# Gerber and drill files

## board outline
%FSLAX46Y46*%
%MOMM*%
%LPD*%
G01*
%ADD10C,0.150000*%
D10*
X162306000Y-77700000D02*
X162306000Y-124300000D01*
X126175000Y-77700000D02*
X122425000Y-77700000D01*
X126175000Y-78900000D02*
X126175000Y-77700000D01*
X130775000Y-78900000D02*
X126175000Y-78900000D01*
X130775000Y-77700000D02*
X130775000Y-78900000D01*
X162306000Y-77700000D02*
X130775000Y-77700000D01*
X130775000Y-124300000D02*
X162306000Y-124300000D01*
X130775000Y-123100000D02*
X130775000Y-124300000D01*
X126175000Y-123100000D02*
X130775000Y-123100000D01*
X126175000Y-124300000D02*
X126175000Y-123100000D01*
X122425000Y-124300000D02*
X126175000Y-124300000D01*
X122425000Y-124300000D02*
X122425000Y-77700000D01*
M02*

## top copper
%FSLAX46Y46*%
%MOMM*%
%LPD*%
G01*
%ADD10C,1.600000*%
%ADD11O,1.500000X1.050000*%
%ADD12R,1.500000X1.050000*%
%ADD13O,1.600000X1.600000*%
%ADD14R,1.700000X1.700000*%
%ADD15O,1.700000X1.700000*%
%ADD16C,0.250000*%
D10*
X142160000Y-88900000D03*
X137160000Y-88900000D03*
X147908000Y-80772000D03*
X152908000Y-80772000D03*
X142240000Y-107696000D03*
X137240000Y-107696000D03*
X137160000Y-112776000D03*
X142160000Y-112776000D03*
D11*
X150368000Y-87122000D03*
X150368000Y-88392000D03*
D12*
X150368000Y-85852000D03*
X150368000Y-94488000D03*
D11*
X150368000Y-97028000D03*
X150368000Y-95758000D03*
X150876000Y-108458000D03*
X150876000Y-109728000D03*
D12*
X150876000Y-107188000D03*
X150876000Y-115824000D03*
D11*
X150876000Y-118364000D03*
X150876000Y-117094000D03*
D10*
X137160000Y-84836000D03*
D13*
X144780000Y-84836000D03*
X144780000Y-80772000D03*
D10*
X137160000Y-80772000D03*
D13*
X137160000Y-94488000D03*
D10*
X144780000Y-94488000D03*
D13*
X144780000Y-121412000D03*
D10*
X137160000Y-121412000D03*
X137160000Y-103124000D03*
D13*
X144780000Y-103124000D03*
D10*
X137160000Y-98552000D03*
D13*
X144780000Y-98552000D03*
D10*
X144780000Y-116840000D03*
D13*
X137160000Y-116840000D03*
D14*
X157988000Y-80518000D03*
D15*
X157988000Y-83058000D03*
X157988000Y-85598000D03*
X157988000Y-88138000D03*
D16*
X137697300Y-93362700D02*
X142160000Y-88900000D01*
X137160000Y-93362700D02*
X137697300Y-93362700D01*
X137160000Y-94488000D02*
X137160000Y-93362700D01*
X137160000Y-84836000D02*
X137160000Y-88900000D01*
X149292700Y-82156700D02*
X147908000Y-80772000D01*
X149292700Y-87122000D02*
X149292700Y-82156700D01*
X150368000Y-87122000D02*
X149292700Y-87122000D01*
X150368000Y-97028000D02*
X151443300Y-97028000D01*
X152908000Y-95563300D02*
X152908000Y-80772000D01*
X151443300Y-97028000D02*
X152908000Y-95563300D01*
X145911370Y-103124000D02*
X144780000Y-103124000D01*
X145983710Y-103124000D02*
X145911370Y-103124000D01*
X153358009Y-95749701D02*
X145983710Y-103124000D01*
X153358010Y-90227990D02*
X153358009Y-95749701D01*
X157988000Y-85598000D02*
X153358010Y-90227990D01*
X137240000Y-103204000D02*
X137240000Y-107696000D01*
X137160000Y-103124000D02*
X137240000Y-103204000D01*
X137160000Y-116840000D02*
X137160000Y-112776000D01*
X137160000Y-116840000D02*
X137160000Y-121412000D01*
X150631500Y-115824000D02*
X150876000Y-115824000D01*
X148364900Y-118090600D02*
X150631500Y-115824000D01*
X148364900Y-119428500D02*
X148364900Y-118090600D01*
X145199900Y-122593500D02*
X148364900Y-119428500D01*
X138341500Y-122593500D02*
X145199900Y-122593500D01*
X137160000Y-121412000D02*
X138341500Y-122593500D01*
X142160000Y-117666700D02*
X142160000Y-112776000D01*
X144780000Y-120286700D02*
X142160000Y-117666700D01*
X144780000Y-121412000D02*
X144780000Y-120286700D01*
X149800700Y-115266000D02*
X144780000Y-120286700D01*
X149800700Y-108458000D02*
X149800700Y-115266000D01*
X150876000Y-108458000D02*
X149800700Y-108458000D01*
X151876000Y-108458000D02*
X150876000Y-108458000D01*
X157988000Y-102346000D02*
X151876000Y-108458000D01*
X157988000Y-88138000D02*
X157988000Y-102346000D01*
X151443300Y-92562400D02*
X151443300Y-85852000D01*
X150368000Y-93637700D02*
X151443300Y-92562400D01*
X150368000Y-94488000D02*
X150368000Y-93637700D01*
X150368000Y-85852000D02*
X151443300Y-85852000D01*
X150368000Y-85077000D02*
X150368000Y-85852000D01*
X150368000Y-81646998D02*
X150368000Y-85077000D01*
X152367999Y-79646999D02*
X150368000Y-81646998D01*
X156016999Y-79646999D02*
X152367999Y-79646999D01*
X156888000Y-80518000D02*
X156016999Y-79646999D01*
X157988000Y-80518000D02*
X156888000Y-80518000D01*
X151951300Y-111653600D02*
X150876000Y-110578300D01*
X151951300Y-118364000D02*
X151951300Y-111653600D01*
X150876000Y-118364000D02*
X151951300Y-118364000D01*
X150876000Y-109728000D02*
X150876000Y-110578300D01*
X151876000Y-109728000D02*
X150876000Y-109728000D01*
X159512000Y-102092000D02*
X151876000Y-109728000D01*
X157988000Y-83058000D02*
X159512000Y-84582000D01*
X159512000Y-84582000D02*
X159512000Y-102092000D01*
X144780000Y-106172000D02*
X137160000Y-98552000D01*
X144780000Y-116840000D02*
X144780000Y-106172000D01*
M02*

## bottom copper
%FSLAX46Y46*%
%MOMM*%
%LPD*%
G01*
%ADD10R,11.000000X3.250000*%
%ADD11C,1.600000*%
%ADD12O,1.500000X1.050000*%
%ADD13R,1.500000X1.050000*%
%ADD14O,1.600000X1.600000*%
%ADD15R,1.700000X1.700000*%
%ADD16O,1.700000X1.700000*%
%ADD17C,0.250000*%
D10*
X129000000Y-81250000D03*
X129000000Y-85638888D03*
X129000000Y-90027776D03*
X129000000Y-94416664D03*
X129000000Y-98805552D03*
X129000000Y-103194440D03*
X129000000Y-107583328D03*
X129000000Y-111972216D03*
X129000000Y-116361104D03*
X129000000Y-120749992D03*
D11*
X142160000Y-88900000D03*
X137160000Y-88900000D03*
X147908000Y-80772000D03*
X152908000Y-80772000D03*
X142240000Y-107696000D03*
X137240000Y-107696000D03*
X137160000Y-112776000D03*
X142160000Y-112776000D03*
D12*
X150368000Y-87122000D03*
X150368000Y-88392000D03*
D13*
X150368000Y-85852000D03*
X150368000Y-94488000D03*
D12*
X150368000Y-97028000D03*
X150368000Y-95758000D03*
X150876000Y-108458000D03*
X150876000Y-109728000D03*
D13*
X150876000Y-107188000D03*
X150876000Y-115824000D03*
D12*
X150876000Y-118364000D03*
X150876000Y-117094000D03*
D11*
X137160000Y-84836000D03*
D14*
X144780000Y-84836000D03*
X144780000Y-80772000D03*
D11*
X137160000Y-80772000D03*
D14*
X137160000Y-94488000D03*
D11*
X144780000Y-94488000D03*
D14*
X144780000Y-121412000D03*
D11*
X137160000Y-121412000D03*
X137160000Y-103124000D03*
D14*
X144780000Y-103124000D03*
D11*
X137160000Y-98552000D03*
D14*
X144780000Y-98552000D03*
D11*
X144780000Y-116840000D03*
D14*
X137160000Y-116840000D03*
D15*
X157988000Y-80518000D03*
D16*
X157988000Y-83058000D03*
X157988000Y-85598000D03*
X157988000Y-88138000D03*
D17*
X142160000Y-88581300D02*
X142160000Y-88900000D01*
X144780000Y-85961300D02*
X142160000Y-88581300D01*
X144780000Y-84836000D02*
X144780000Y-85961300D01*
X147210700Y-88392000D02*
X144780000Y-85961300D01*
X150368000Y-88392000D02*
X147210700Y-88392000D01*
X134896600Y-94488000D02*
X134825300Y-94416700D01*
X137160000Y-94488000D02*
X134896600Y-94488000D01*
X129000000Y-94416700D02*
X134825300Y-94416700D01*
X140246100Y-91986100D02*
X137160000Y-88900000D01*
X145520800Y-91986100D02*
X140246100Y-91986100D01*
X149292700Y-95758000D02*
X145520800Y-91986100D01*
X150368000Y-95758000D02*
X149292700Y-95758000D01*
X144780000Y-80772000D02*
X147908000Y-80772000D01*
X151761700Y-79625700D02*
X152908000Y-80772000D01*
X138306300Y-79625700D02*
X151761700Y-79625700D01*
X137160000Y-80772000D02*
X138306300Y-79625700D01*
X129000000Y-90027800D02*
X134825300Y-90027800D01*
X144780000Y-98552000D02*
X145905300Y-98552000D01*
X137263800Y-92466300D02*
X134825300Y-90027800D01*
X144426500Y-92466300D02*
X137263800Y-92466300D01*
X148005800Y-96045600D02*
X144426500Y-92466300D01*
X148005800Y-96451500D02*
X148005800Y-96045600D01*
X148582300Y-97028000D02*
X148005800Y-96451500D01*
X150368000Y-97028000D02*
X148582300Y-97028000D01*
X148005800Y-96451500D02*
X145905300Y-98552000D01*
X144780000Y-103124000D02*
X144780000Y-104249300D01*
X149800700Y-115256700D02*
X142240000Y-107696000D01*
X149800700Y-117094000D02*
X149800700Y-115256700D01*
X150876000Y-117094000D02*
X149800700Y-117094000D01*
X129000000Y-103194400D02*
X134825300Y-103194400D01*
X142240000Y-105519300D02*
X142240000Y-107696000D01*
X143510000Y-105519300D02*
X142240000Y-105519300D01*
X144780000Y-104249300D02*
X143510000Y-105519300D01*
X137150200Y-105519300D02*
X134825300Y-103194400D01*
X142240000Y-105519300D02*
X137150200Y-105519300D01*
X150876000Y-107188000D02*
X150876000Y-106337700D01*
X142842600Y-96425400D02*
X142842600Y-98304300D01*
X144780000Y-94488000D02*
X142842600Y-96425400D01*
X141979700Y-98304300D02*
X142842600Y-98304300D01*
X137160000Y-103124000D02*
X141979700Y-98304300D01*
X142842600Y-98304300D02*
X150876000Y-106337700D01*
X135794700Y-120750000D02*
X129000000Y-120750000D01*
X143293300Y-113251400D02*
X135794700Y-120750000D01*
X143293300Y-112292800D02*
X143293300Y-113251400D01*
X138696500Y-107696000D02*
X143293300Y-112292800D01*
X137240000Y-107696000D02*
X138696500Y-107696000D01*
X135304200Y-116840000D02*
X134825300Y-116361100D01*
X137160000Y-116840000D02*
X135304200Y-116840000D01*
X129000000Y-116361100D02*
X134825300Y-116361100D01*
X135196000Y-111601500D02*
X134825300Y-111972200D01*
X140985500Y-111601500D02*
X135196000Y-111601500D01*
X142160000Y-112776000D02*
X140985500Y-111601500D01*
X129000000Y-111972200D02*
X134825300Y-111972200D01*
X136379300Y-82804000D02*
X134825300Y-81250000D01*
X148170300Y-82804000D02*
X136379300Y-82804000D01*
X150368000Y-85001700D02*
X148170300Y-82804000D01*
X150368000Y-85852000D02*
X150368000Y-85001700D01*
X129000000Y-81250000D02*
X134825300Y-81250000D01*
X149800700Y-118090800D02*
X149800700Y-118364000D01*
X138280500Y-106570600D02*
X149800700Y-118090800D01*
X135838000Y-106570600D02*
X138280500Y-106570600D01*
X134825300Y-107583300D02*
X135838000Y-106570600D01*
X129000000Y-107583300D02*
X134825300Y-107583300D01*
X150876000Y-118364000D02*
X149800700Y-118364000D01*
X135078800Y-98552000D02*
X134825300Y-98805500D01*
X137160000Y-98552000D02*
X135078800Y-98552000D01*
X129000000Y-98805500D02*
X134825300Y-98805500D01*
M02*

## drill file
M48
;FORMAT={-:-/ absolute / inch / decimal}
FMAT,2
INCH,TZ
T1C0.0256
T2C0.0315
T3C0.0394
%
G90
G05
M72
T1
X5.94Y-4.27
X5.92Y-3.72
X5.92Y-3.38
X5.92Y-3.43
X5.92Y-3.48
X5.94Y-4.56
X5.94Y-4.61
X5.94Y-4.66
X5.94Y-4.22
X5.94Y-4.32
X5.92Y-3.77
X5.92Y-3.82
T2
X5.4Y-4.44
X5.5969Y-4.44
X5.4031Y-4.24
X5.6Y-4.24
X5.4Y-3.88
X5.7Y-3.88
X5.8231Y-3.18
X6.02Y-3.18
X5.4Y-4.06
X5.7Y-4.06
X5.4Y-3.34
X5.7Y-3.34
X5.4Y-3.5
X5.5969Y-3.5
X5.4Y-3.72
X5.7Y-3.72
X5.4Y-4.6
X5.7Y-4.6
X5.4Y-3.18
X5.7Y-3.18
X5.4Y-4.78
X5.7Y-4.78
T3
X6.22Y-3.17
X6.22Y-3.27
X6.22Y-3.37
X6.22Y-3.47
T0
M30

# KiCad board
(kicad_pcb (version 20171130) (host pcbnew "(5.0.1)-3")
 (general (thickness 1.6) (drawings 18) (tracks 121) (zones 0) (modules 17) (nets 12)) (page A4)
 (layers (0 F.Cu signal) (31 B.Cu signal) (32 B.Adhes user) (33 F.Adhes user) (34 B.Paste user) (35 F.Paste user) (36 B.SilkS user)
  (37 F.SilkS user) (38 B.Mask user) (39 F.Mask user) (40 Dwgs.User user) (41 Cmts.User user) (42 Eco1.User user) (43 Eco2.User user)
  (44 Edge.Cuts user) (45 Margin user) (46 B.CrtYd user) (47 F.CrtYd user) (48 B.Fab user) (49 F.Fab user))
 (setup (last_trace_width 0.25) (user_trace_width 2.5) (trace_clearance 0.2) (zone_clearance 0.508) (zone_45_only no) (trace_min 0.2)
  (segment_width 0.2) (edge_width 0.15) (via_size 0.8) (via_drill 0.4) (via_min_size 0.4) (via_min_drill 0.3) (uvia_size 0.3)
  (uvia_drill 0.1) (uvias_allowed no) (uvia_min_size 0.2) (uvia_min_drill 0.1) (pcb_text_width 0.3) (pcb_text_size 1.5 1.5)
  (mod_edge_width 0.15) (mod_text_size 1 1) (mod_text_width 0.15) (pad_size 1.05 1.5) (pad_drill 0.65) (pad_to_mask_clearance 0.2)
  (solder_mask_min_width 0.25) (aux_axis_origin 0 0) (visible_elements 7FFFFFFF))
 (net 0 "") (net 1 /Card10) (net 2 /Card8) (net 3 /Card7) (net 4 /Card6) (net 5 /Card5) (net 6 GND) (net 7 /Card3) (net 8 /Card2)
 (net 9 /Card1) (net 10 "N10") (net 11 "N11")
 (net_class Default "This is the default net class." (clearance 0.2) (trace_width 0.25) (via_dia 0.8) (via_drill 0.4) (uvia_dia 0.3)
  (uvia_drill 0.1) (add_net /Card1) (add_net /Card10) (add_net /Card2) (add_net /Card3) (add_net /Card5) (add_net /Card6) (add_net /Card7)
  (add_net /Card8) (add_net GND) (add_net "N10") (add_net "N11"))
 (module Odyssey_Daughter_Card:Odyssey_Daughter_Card (layer F.Cu) (at 129 101)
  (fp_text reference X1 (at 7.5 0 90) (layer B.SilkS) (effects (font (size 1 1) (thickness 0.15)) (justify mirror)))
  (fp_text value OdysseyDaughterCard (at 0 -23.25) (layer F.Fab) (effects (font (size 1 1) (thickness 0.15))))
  (pad 10 smd rect (at 0 -19.75) (size 11 3.25) (layers B.Cu B.Mask) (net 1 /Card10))
  (pad 9 smd rect (at 0 -15.361112) (size 11 3.25) (layers B.Cu B.Mask))
  (pad 8 smd rect (at 0 -10.972224) (size 11 3.25) (layers B.Cu B.Mask) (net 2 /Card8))
  (pad 7 smd rect (at 0 -6.583336) (size 11 3.25) (layers B.Cu B.Mask) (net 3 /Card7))
  (pad 6 smd rect (at 0 -2.194448) (size 11 3.25) (layers B.Cu B.Mask) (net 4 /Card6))
  (pad 5 smd rect (at 0 2.19444) (size 11 3.25) (layers B.Cu B.Mask) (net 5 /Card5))
  (pad 4 smd rect (at 0 6.583328) (size 11 3.25) (layers B.Cu B.Mask) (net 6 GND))
  (pad 3 smd rect (at 0 10.972216) (size 11 3.25) (layers B.Cu B.Mask) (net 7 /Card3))
  (pad 2 smd rect (at 0 15.361104) (size 11 3.25) (layers B.Cu B.Mask) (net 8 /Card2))
  (pad 1 smd rect (at 0 19.749992) (size 11 3.25) (layers B.Cu B.Mask) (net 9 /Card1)))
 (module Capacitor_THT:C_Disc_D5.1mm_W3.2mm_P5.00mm (layer F.Cu) (at 137.16 88.9)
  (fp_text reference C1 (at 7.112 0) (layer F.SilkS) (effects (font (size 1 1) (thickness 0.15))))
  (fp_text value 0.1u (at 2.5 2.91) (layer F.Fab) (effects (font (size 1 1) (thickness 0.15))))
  (pad 2 thru_hole circle (at 5 0) (size 1.6 1.6) (drill 0.8) (layers *.Cu *.Mask) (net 3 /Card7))
  (pad 1 thru_hole circle (at 0 0) (size 1.6 1.6) (drill 0.8) (layers *.Cu *.Mask) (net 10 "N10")))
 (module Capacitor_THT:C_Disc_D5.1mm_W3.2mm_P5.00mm (layer F.Cu) (at 152.908 80.772 180)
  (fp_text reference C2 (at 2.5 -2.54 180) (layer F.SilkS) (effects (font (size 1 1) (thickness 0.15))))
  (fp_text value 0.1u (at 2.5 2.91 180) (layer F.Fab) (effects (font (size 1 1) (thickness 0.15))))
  (pad 2 thru_hole circle (at 5 0 180) (size 1.6 1.6) (drill 0.8) (layers *.Cu *.Mask) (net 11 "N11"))
  (pad 1 thru_hole circle (at 0 0 180) (size 1.6 1.6) (drill 0.8) (layers *.Cu *.Mask) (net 2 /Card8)))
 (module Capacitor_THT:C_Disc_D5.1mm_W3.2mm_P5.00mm (layer F.Cu) (at 142.24 107.696 180)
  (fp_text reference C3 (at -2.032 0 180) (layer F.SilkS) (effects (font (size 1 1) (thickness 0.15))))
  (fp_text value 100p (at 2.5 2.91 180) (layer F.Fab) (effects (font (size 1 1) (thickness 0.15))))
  (pad 1 thru_hole circle (at 0 0 180) (size 1.6 1.6) (drill 0.8) (layers *.Cu *.Mask) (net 5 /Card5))
  (pad 2 thru_hole circle (at 5 0 180) (size 1.6 1.6) (drill 0.8) (layers *.Cu *.Mask) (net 9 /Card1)))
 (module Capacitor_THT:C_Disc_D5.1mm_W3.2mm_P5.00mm (layer F.Cu) (at 137.16 112.776)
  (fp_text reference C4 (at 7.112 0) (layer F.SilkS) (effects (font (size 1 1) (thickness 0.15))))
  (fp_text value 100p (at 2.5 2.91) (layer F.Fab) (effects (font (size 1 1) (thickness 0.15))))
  (pad 1 thru_hole circle (at 0 0) (size 1.6 1.6) (drill 0.8) (layers *.Cu *.Mask) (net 8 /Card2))
  (pad 2 thru_hole circle (at 5 0) (size 1.6 1.6) (drill 0.8) (layers *.Cu *.Mask) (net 7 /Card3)))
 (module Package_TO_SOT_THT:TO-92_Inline (layer F.Cu) (at 150.368 85.852 270)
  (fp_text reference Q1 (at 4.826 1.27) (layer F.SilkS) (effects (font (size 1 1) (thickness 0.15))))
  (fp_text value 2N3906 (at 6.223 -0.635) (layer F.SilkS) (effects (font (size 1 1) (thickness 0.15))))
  (pad 2 thru_hole oval (at 1.27 0 270) (size 1.05 1.5) (drill 0.65) (layers *.Cu *.Mask) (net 11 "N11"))
  (pad 3 thru_hole oval (at 2.54 0 270) (size 1.05 1.5) (drill 0.65) (layers *.Cu *.Mask) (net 3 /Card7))
  (pad 1 thru_hole rect (at 0 0 270) (size 1.05 1.5) (drill 0.65) (layers *.Cu *.Mask) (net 1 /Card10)))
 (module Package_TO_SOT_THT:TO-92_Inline (layer F.Cu) (at 150.368 94.488 270)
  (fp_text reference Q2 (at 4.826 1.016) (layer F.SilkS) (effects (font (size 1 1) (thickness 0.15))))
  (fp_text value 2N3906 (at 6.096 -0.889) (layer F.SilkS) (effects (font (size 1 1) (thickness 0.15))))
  (pad 1 thru_hole rect (at 0 0 270) (size 1.05 1.5) (drill 0.65) (layers *.Cu *.Mask) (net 1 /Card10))
  (pad 3 thru_hole oval (at 2.54 0 270) (size 1.05 1.5) (drill 0.65) (layers *.Cu *.Mask) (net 2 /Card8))
  (pad 2 thru_hole oval (at 1.27 0 270) (size 1.05 1.5) (drill 0.65) (layers *.Cu *.Mask) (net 10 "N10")))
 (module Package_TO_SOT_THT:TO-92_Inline (layer F.Cu) (at 150.876 107.188 270)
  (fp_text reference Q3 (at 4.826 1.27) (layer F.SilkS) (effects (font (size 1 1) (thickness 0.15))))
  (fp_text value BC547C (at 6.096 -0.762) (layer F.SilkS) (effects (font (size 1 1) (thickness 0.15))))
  (pad 2 thru_hole oval (at 1.27 0 270) (size 1.05 1.5) (drill 0.65) (layers *.Cu *.Mask) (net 7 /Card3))
  (pad 3 thru_hole oval (at 2.54 0 270) (size 1.05 1.5) (drill 0.65) (layers *.Cu *.Mask) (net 6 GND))
  (pad 1 thru_hole rect (at 0 0 270) (size 1.05 1.5) (drill 0.65) (layers *.Cu *.Mask) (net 9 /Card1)))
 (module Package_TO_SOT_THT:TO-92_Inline (layer F.Cu) (at 150.876 115.824 270)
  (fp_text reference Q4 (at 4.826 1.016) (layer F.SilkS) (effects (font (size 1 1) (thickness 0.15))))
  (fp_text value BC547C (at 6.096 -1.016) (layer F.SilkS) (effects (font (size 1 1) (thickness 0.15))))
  (pad 1 thru_hole rect (at 0 0 270) (size 1.05 1.5) (drill 0.65) (layers *.Cu *.Mask) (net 8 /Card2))
  (pad 3 thru_hole oval (at 2.54 0 270) (size 1.05 1.5) (drill 0.65) (layers *.Cu *.Mask) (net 6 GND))
  (pad 2 thru_hole oval (at 1.27 0 270) (size 1.05 1.5) (drill 0.65) (layers *.Cu *.Mask) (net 5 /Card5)))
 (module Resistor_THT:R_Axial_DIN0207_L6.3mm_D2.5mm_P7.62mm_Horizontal (layer F.Cu) (at 137.16 84.836)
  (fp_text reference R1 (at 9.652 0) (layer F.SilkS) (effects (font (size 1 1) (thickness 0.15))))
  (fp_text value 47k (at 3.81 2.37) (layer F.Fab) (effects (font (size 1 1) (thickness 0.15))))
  (pad 1 thru_hole circle (at 0 0) (size 1.6 1.6) (drill 0.8) (layers *.Cu *.Mask) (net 10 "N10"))
  (pad 2 thru_hole oval (at 7.62 0) (size 1.6 1.6) (drill 0.8) (layers *.Cu *.Mask) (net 3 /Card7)))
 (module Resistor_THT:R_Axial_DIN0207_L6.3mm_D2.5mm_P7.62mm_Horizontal (layer F.Cu) (at 137.16 80.772)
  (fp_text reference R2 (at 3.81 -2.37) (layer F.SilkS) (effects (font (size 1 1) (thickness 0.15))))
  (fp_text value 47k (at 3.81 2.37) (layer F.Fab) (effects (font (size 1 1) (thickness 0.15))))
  (pad 2 thru_hole oval (at 7.62 0) (size 1.6 1.6) (drill 0.8) (layers *.Cu *.Mask) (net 11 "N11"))
  (pad 1 thru_hole circle (at 0 0) (size 1.6 1.6) (drill 0.8) (layers *.Cu *.Mask) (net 2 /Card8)))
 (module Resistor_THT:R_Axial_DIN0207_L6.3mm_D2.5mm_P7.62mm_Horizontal (layer F.Cu) (at 144.78 94.488 180)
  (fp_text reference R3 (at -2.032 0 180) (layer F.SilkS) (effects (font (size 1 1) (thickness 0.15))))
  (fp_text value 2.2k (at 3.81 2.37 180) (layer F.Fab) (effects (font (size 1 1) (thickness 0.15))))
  (pad 2 thru_hole oval (at 7.62 0 180) (size 1.6 1.6) (drill 0.8) (layers *.Cu *.Mask) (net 3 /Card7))
  (pad 1 thru_hole circle (at 0 0 180) (size 1.6 1.6) (drill 0.8) (layers *.Cu *.Mask) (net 9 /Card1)))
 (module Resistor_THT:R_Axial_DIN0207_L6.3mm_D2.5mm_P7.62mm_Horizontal (layer F.Cu) (at 137.16 121.412)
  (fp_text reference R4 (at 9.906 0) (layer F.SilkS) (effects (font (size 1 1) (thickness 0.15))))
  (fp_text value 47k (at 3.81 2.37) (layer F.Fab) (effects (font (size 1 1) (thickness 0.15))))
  (pad 2 thru_hole oval (at 7.62 0) (size 1.6 1.6) (drill 0.8) (layers *.Cu *.Mask) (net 7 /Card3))
  (pad 1 thru_hole circle (at 0 0) (size 1.6 1.6) (drill 0.8) (layers *.Cu *.Mask) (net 8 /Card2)))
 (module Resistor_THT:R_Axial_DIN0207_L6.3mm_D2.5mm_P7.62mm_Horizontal (layer F.Cu) (at 137.16 103.124)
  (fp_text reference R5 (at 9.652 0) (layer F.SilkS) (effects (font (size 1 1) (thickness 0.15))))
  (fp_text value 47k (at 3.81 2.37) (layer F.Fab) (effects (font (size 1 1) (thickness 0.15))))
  (pad 1 thru_hole circle (at 0 0) (size 1.6 1.6) (drill 0.8) (layers *.Cu *.Mask) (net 9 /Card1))
  (pad 2 thru_hole oval (at 7.62 0) (size 1.6 1.6) (drill 0.8) (layers *.Cu *.Mask) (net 5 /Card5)))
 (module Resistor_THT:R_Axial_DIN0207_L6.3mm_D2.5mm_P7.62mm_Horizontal (layer F.Cu) (at 137.16 98.552)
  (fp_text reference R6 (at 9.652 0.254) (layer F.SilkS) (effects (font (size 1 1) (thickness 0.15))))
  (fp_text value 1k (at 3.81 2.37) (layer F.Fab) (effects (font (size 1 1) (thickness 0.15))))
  (pad 1 thru_hole circle (at 0 0) (size 1.6 1.6) (drill 0.8) (layers *.Cu *.Mask) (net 4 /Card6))
  (pad 2 thru_hole oval (at 7.62 0) (size 1.6 1.6) (drill 0.8) (layers *.Cu *.Mask) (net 2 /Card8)))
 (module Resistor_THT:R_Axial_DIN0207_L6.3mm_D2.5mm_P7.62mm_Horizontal (layer F.Cu) (at 144.78 116.84 180)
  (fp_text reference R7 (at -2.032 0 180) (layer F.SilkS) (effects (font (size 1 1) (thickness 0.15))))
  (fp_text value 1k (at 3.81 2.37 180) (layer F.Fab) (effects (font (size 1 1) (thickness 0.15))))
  (pad 1 thru_hole circle (at 0 0 180) (size 1.6 1.6) (drill 0.8) (layers *.Cu *.Mask) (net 4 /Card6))
  (pad 2 thru_hole oval (at 7.62 0 180) (size 1.6 1.6) (drill 0.8) (layers *.Cu *.Mask) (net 8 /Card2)))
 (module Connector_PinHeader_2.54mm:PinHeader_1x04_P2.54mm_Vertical (layer F.Cu) (at 157.988 80.518)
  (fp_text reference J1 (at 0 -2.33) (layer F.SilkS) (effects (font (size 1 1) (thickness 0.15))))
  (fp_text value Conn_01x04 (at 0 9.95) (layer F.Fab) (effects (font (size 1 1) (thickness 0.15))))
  (pad 1 thru_hole rect (at 0 0) (size 1.7 1.7) (drill 1) (layers *.Cu *.Mask) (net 1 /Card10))
  (pad 2 thru_hole oval (at 0 2.54) (size 1.7 1.7) (drill 1) (layers *.Cu *.Mask) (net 6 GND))
  (pad 3 thru_hole oval (at 0 5.08) (size 1.7 1.7) (drill 1) (layers *.Cu *.Mask) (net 5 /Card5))
  (pad 4 thru_hole oval (at 0 7.62) (size 1.7 1.7) (drill 1) (layers *.Cu *.Mask) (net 7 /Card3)))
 (gr_line (start 162.306 77.7) (end 162.306 124.3) (layer Edge.Cuts) (width 0.15))
 (gr_line (start 126.175 77.7) (end 122.425 77.7) (layer Edge.Cuts) (width 0.15))
 (gr_line (start 126.175 78.9) (end 126.175 77.7) (layer Edge.Cuts) (width 0.15))
 (gr_line (start 130.775 78.9) (end 126.175 78.9) (layer Edge.Cuts) (width 0.15))
 (gr_line (start 130.775 77.7) (end 130.775 78.9) (layer Edge.Cuts) (width 0.15))
 (gr_line (start 162.306 77.7) (end 130.775 77.7) (layer Edge.Cuts) (width 0.15))
 (gr_line (start 130.775 124.3) (end 162.306 124.3) (layer Edge.Cuts) (width 0.15))
 (gr_line (start 130.775 123.1) (end 130.775 124.3) (layer Edge.Cuts) (width 0.15))
 (gr_line (start 126.175 123.1) (end 130.775 123.1) (layer Edge.Cuts) (width 0.15))
 (gr_line (start 126.175 124.3) (end 126.175 123.1) (layer Edge.Cuts) (width 0.15))
 (gr_line (start 122.425 124.3) (end 126.175 124.3) (layer Edge.Cuts) (width 0.15))
 (gr_line (start 122.425 124.3) (end 122.425 77.7) (layer Edge.Cuts) (width 0.15))
 (segment (start 142.16 88.5813) (end 142.16 88.9) (width 0.25) (layer B.Cu) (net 3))
 (segment (start 144.78 85.9613) (end 142.16 88.5813) (width 0.25) (layer B.Cu) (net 3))
 (segment (start 144.78 84.836) (end 144.78 85.9613) (width 0.25) (layer B.Cu) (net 3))
 (segment (start 147.2107 88.392) (end 144.78 85.9613) (width 0.25) (layer B.Cu) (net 3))
 (segment (start 150.368 88.392) (end 147.2107 88.392) (width 0.25) (layer B.Cu) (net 3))
 (segment (start 134.8966 94.488) (end 134.8253 94.4167) (width 0.25) (layer B.Cu) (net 3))
 (segment (start 137.16 94.488) (end 134.8966 94.488) (width 0.25) (layer B.Cu) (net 3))
 (segment (start 129 94.4167) (end 134.8253 94.4167) (width 0.25) (layer B.Cu) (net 3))
 (segment (start 137.6973 93.3627) (end 142.16 88.9) (width 0.25) (layer F.Cu) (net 3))
 (segment (start 137.16 93.3627) (end 137.6973 93.3627) (width 0.25) (layer F.Cu) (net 3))
 (segment (start 137.16 94.488) (end 137.16 93.3627) (width 0.25) (layer F.Cu) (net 3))
 (segment (start 137.16 84.836) (end 137.16 88.9) (width 0.25) (layer F.Cu) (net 10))
 (segment (start 140.2461 91.9861) (end 137.16 88.9) (width 0.25) (layer B.Cu) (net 10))
 (segment (start 145.5208 91.9861) (end 140.2461 91.9861) (width 0.25) (layer B.Cu) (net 10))
 (segment (start 149.2927 95.758) (end 145.5208 91.9861) (width 0.25) (layer B.Cu) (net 10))
 (segment (start 150.368 95.758) (end 149.2927 95.758) (width 0.25) (layer B.Cu) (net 10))
 (segment (start 144.78 80.772) (end 147.908 80.772) (width 0.25) (layer B.Cu) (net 11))
 (segment (start 149.2927 82.1567) (end 147.908 80.772) (width 0.25) (layer F.Cu) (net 11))
 (segment (start 149.2927 87.122) (end 149.2927 82.1567) (width 0.25) (layer F.Cu) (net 11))
 (segment (start 150.368 87.122) (end 149.2927 87.122) (width 0.25) (layer F.Cu) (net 11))
 (segment (start 151.7617 79.6257) (end 152.908 80.772) (width 0.25) (layer B.Cu) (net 2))
 (segment (start 138.3063 79.6257) (end 151.7617 79.6257) (width 0.25) (layer B.Cu) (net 2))
 (segment (start 137.16 80.772) (end 138.3063 79.6257) (width 0.25) (layer B.Cu) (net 2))
 (segment (start 150.368 97.028) (end 151.4433 97.028) (width 0.25) (layer F.Cu) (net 2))
 (segment (start 152.908 95.5633) (end 152.908 80.772) (width 0.25) (layer F.Cu) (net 2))
 (segment (start 151.4433 97.028) (end 152.908 95.5633) (width 0.25) (layer F.Cu) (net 2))
 (segment (start 129 90.0278) (end 134.8253 90.0278) (width 0.25) (layer B.Cu) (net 2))
 (segment (start 144.78 98.552) (end 145.9053 98.552) (width 0.25) (layer B.Cu) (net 2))
 (segment (start 137.2638 92.4663) (end 134.8253 90.0278) (width 0.25) (layer B.Cu) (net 2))
 (segment (start 144.4265 92.4663) (end 137.2638 92.4663) (width 0.25) (layer B.Cu) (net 2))
 (segment (start 148.0058 96.0456) (end 144.4265 92.4663) (width 0.25) (layer B.Cu) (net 2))
 (segment (start 148.0058 96.4515) (end 148.0058 96.0456) (width 0.25) (layer B.Cu) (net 2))
 (segment (start 148.5823 97.028) (end 148.0058 96.4515) (width 0.25) (layer B.Cu) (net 2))
 (segment (start 150.368 97.028) (end 148.5823 97.028) (width 0.25) (layer B.Cu) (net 2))
 (segment (start 148.0058 96.4515) (end 145.9053 98.552) (width 0.25) (layer B.Cu) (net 2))
 (segment (start 144.78 103.124) (end 144.78 104.2493) (width 0.25) (layer B.Cu) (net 5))
 (segment (start 149.8007 115.2567) (end 142.24 107.696) (width 0.25) (layer B.Cu) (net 5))
 (segment (start 149.8007 117.094) (end 149.8007 115.2567) (width 0.25) (layer B.Cu) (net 5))
 (segment (start 150.876 117.094) (end 149.8007 117.094) (width 0.25) (layer B.Cu) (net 5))
 (segment (start 129 103.1944) (end 134.8253 103.1944) (width 0.25) (layer B.Cu) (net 5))
 (segment (start 142.24 105.5193) (end 142.24 107.696) (width 0.25) (layer B.Cu) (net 5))
 (segment (start 143.51 105.5193) (end 142.24 105.5193) (width 0.25) (layer B.Cu) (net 5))
 (segment (start 144.78 104.2493) (end 143.51 105.5193) (width 0.25) (layer B.Cu) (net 5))
 (segment (start 137.1502 105.5193) (end 134.8253 103.1944) (width 0.25) (layer B.Cu) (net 5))
 (segment (start 142.24 105.5193) (end 137.1502 105.5193) (width 0.25) (layer B.Cu) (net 5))
 (segment (start 145.91137 103.124) (end 144.78 103.124) (width 0.25) (layer F.Cu) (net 5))
 (segment (start 145.98371 103.124) (end 145.91137 103.124) (width 0.25) (layer F.Cu) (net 5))
 (segment (start 153.358009 95.749701) (end 145.98371 103.124) (width 0.25) (layer F.Cu) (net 5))
 (segment (start 153.35801 90.22799) (end 153.358009 95.749701) (width 0.25) (layer F.Cu) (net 5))
 (segment (start 157.988 85.598) (end 153.35801 90.22799) (width 0.25) (layer F.Cu) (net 5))
 (segment (start 137.24 103.204) (end 137.24 107.696) (width 0.25) (layer F.Cu) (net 9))
 (segment (start 137.16 103.124) (end 137.24 103.204) (width 0.25) (layer F.Cu) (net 9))
 (segment (start 150.876 107.188) (end 150.876 106.3377) (width 0.25) (layer B.Cu) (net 9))
 (segment (start 142.8426 96.4254) (end 142.8426 98.3043) (width 0.25) (layer B.Cu) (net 9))
 (segment (start 144.78 94.488) (end 142.8426 96.4254) (width 0.25) (layer B.Cu) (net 9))
 (segment (start 141.9797 98.3043) (end 142.8426 98.3043) (width 0.25) (layer B.Cu) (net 9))
 (segment (start 137.16 103.124) (end 141.9797 98.3043) (width 0.25) (layer B.Cu) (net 9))
 (segment (start 142.8426 98.3043) (end 150.876 106.3377) (width 0.25) (layer B.Cu) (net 9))
 (segment (start 135.7947 120.75) (end 129 120.75) (width 0.25) (layer B.Cu) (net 9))
 (segment (start 143.2933 113.2514) (end 135.7947 120.75) (width 0.25) (layer B.Cu) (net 9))
 (segment (start 143.2933 112.2928) (end 143.2933 113.2514) (width 0.25) (layer B.Cu) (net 9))
 (segment (start 138.6965 107.696) (end 143.2933 112.2928) (width 0.25) (layer B.Cu) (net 9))
 (segment (start 137.24 107.696) (end 138.6965 107.696) (width 0.25) (layer B.Cu) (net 9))
 (segment (start 137.16 116.84) (end 137.16 112.776) (width 0.25) (layer F.Cu) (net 8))
 (segment (start 135.3042 116.84) (end 134.8253 116.3611) (width 0.25) (layer B.Cu) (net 8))
 (segment (start 137.16 116.84) (end 135.3042 116.84) (width 0.25) (layer B.Cu) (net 8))
 (segment (start 129 116.3611) (end 134.8253 116.3611) (width 0.25) (layer B.Cu) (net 8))
 (segment (start 137.16 116.84) (end 137.16 121.412) (width 0.25) (layer F.Cu) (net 8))
 (segment (start 150.6315 115.824) (end 150.876 115.824) (width 0.25) (layer F.Cu) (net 8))
 (segment (start 148.3649 118.0906) (end 150.6315 115.824) (width 0.25) (layer F.Cu) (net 8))
 (segment (start 148.3649 119.4285) (end 148.3649 118.0906) (width 0.25) (layer F.Cu) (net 8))
 (segment (start 145.1999 122.5935) (end 148.3649 119.4285) (width 0.25) (layer F.Cu) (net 8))
 (segment (start 138.3415 122.5935) (end 145.1999 122.5935) (width 0.25) (layer F.Cu) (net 8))
 (segment (start 137.16 121.412) (end 138.3415 122.5935) (width 0.25) (layer F.Cu) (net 8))
 (segment (start 142.16 117.6667) (end 142.16 112.776) (width 0.25) (layer F.Cu) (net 7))
 (segment (start 144.78 120.2867) (end 142.16 117.6667) (width 0.25) (layer F.Cu) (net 7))
 (segment (start 144.78 121.412) (end 144.78 120.2867) (width 0.25) (layer F.Cu) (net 7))
 (segment (start 149.8007 115.266) (end 144.78 120.2867) (width 0.25) (layer F.Cu) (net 7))
 (segment (start 149.8007 108.458) (end 149.8007 115.266) (width 0.25) (layer F.Cu) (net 7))
 (segment (start 150.876 108.458) (end 149.8007 108.458) (width 0.25) (layer F.Cu) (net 7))
 (segment (start 135.196 111.6015) (end 134.8253 111.9722) (width 0.25) (layer B.Cu) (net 7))
 (segment (start 140.9855 111.6015) (end 135.196 111.6015) (width 0.25) (layer B.Cu) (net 7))
 (segment (start 142.16 112.776) (end 140.9855 111.6015) (width 0.25) (layer B.Cu) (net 7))
 (segment (start 129 111.9722) (end 134.8253 111.9722) (width 0.25) (layer B.Cu) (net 7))
 (segment (start 151.876 108.458) (end 150.876 108.458) (width 0.25) (layer F.Cu) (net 7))
 (segment (start 157.988 102.346) (end 151.876 108.458) (width 0.25) (layer F.Cu) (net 7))
 (segment (start 157.988 88.138) (end 157.988 102.346) (width 0.25) (layer F.Cu) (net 7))
 (segment (start 151.4433 92.5624) (end 151.4433 85.852) (width 0.25) (layer F.Cu) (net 1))
 (segment (start 150.368 93.6377) (end 151.4433 92.5624) (width 0.25) (layer F.Cu) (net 1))
 (segment (start 150.368 94.488) (end 150.368 93.6377) (width 0.25) (layer F.Cu) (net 1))
 (segment (start 150.368 85.852) (end 151.4433 85.852) (width 0.25) (layer F.Cu) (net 1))
 (segment (start 136.3793 82.804) (end 134.8253 81.25) (width 0.25) (layer B.Cu) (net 1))
 (segment (start 148.1703 82.804) (end 136.3793 82.804) (width 0.25) (layer B.Cu) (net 1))
 (segment (start 150.368 85.0017) (end 148.1703 82.804) (width 0.25) (layer B.Cu) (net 1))
 (segment (start 150.368 85.852) (end 150.368 85.0017) (width 0.25) (layer B.Cu) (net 1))
 (segment (start 129 81.25) (end 134.8253 81.25) (width 0.25) (layer B.Cu) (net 1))
 (segment (start 150.368 85.077) (end 150.368 85.852) (width 0.25) (layer F.Cu) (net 1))
 (segment (start 150.368 81.646998) (end 150.368 85.077) (width 0.25) (layer F.Cu) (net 1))
 (segment (start 152.367999 79.646999) (end 150.368 81.646998) (width 0.25) (layer F.Cu) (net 1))
 (segment (start 156.016999 79.646999) (end 152.367999 79.646999) (width 0.25) (layer F.Cu) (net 1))
 (segment (start 156.888 80.518) (end 156.016999 79.646999) (width 0.25) (layer F.Cu) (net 1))
 (segment (start 157.988 80.518) (end 156.888 80.518) (width 0.25) (layer F.Cu) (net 1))
 (segment (start 151.9513 111.6536) (end 150.876 110.5783) (width 0.25) (layer F.Cu) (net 6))
 (segment (start 151.9513 118.364) (end 151.9513 111.6536) (width 0.25) (layer F.Cu) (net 6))
 (segment (start 150.876 118.364) (end 151.9513 118.364) (width 0.25) (layer F.Cu) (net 6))
 (segment (start 150.876 109.728) (end 150.876 110.5783) (width 0.25) (layer F.Cu) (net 6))
 (segment (start 149.8007 118.0908) (end 149.8007 118.364) (width 0.25) (layer B.Cu) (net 6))
 (segment (start 138.2805 106.5706) (end 149.8007 118.0908) (width 0.25) (layer B.Cu) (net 6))
 (segment (start 135.838 106.5706) (end 138.2805 106.5706) (width 0.25) (layer B.Cu) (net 6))
 (segment (start 134.8253 107.5833) (end 135.838 106.5706) (width 0.25) (layer B.Cu) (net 6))
 (segment (start 129 107.5833) (end 134.8253 107.5833) (width 0.25) (layer B.Cu) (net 6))
 (segment (start 150.876 118.364) (end 149.8007 118.364) (width 0.25) (layer B.Cu) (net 6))
 (segment (start 151.876 109.728) (end 150.876 109.728) (width 0.25) (layer F.Cu) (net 6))
 (segment (start 159.512 102.092) (end 151.876 109.728) (width 0.25) (layer F.Cu) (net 6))
 (segment (start 157.988 83.058) (end 159.512 84.582) (width 0.25) (layer F.Cu) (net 6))
 (segment (start 159.512 84.582) (end 159.512 102.092) (width 0.25) (layer F.Cu) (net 6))
 (segment (start 144.78 106.172) (end 137.16 98.552) (width 0.25) (layer F.Cu) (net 4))
 (segment (start 144.78 116.84) (end 144.78 106.172) (width 0.25) (layer F.Cu) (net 4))
 (segment (start 135.0788 98.552) (end 134.8253 98.8055) (width 0.25) (layer B.Cu) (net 4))
 (segment (start 137.16 98.552) (end 135.0788 98.552) (width 0.25) (layer B.Cu) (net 4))
 (segment (start 129 98.8055) (end 134.8253 98.8055) (width 0.25) (layer B.Cu) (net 4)))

